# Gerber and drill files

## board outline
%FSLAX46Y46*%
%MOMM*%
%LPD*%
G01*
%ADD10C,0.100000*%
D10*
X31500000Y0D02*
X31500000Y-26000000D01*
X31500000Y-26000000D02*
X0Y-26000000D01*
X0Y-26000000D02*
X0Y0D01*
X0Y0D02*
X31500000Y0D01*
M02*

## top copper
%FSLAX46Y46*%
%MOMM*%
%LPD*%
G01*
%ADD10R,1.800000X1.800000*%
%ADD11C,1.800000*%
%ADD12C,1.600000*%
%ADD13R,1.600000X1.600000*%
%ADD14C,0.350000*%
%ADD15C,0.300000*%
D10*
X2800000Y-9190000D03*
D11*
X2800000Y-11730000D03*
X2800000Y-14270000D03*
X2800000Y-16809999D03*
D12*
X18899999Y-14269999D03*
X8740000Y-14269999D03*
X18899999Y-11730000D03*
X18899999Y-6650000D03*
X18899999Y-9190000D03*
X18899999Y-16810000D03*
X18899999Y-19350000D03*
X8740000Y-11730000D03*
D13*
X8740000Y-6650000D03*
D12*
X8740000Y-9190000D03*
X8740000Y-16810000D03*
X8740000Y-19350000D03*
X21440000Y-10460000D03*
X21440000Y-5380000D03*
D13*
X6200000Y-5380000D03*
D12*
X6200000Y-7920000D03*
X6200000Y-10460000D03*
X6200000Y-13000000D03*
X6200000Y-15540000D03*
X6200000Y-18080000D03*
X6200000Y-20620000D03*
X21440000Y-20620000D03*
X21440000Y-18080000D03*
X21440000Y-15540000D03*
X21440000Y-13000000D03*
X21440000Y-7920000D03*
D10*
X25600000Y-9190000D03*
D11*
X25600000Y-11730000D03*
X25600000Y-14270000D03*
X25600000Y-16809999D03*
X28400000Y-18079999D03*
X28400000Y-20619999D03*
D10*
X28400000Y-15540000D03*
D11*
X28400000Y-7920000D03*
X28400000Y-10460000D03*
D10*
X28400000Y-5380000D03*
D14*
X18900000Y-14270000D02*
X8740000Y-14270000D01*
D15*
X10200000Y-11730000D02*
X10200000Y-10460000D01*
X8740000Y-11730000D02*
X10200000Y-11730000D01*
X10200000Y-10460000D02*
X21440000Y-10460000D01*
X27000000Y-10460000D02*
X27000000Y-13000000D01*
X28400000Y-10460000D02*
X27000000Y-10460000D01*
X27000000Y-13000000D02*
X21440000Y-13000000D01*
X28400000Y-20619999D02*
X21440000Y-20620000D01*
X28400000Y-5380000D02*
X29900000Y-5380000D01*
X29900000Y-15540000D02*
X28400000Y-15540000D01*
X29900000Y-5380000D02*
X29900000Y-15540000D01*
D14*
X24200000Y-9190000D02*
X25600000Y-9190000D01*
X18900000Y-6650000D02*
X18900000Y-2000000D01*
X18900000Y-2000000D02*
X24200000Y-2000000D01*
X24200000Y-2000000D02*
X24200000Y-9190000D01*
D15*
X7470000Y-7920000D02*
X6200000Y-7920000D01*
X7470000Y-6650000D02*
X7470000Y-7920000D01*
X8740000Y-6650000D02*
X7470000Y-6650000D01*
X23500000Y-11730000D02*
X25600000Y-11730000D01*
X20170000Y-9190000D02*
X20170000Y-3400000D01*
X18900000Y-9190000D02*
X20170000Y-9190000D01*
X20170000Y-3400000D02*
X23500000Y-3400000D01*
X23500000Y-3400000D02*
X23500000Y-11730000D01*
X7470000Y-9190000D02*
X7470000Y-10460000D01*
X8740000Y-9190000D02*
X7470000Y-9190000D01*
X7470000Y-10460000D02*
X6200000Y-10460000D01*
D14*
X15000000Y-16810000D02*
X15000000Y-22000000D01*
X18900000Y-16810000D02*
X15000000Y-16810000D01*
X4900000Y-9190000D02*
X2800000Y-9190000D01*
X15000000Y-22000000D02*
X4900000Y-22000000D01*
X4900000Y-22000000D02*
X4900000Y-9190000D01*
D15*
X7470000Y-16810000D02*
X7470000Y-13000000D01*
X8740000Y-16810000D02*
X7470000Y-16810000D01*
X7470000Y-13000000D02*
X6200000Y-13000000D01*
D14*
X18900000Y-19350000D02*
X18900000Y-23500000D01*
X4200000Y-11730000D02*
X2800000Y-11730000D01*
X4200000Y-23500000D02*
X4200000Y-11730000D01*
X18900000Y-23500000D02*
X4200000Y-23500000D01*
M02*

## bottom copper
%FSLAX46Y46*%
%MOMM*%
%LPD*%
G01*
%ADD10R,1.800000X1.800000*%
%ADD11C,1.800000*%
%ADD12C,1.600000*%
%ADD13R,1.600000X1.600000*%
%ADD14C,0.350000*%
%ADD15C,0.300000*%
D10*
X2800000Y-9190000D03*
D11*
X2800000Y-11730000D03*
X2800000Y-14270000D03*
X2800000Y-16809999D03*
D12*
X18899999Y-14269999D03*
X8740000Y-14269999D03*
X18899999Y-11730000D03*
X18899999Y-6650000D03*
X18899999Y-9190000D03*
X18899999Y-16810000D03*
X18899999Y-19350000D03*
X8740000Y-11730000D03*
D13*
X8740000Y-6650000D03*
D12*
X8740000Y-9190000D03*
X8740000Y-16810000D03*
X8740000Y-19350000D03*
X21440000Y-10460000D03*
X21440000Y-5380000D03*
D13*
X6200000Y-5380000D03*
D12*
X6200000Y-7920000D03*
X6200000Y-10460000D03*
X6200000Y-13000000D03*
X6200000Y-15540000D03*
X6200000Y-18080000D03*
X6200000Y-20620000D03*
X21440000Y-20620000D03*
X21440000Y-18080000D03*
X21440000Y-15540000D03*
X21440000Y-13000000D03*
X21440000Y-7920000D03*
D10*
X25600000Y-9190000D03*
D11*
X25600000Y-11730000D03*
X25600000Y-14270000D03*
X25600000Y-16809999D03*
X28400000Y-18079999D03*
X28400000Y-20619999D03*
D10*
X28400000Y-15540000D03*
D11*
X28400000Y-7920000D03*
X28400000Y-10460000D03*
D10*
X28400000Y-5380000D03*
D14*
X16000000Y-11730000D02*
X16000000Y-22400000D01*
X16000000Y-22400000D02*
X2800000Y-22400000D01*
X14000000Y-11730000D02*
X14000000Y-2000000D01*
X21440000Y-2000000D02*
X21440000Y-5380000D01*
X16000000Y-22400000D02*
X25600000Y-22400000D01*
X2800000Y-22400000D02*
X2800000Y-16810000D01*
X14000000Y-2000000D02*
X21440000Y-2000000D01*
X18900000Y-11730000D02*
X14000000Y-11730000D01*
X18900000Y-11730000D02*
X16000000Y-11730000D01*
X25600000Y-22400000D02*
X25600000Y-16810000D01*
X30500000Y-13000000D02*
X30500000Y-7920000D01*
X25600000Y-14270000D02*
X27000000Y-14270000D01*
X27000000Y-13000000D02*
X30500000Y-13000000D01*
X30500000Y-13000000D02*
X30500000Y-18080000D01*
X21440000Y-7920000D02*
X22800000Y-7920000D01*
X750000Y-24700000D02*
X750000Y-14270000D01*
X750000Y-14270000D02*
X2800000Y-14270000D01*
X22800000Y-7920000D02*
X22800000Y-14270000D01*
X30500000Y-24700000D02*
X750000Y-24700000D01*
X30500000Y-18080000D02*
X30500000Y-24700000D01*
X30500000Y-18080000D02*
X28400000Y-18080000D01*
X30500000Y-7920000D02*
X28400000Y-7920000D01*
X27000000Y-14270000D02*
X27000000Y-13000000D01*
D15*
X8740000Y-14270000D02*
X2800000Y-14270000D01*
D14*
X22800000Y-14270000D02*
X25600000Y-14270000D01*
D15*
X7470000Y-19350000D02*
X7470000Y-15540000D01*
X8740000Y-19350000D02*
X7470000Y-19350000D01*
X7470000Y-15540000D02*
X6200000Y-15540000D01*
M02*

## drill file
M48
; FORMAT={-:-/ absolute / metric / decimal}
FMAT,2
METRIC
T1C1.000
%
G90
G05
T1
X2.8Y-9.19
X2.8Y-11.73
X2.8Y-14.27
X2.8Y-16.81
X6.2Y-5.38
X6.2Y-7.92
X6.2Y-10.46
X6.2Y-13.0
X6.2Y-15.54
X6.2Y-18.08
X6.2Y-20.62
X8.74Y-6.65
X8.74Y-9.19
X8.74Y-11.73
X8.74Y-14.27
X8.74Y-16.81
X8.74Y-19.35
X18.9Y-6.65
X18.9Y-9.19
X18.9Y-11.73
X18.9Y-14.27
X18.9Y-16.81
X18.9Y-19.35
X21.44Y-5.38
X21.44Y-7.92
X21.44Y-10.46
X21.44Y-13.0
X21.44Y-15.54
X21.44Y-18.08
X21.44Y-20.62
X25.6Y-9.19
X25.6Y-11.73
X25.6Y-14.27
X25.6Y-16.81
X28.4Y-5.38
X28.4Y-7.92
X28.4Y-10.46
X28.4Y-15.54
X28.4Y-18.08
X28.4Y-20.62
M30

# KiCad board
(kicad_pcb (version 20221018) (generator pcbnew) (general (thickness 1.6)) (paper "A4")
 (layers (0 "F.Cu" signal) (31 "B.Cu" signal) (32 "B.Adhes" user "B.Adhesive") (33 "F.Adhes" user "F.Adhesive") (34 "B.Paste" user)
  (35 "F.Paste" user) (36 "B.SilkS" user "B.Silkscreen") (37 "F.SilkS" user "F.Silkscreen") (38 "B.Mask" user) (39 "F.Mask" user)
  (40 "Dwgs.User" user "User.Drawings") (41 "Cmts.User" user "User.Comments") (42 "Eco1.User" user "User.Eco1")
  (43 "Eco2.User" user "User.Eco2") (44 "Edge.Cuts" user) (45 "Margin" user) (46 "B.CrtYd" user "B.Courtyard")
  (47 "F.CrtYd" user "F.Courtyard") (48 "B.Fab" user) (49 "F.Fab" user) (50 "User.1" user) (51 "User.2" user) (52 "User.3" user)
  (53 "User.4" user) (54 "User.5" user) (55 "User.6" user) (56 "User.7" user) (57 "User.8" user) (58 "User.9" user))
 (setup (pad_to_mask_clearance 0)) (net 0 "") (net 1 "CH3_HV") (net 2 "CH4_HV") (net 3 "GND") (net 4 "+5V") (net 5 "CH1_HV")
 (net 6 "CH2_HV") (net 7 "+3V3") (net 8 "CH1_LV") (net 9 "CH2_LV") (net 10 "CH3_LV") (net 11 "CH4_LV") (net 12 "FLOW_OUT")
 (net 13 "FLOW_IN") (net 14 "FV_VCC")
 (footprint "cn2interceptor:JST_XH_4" (layer "F.Cu") (at 2.8 9.19)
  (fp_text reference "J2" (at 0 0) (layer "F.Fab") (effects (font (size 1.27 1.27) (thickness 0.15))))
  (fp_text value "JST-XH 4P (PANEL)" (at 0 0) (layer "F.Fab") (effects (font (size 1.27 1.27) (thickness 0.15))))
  (pad "1" thru_hole rect (at 0 0) (size 1.8 1.8) (drill 1) (layers "*.Cu" "*.Mask") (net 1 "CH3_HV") (thermal_bridge_angle 45))
  (pad "2" thru_hole circle (at 0 2.54) (size 1.8 1.8) (drill 1) (layers "*.Cu" "*.Mask") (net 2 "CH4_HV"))
  (pad "3" thru_hole circle (at 0 5.08) (size 1.8 1.8) (drill 1) (layers "*.Cu" "*.Mask") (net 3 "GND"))
  (pad "4" thru_hole circle (at 0 7.619999) (size 1.8 1.8) (drill 1) (layers "*.Cu" "*.Mask") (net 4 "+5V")))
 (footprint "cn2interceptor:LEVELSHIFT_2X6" (layer "F.Cu") (at 8.74 6.65)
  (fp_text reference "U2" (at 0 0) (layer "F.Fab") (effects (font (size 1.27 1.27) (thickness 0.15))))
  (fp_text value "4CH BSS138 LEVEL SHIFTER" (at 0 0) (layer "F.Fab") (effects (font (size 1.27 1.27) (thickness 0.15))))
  (pad "GND_H" thru_hole circle (at 10.159999 7.619999) (size 1.6 1.6) (drill 1) (layers "*.Cu" "*.Mask") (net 3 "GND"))
  (pad "GND_L" thru_hole circle (at 0 7.619999) (size 1.6 1.6) (drill 1) (layers "*.Cu" "*.Mask") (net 3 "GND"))
  (pad "HV" thru_hole circle (at 10.159999 5.08) (size 1.6 1.6) (drill 1) (layers "*.Cu" "*.Mask") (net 4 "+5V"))
  (pad "HV1" thru_hole circle (at 10.159999 0) (size 1.6 1.6) (drill 1) (layers "*.Cu" "*.Mask") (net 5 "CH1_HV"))
  (pad "HV2" thru_hole circle (at 10.159999 2.54) (size 1.6 1.6) (drill 1) (layers "*.Cu" "*.Mask") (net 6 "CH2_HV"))
  (pad "HV3" thru_hole circle (at 10.159999 10.16) (size 1.6 1.6) (drill 1) (layers "*.Cu" "*.Mask") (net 1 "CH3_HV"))
  (pad "HV4" thru_hole circle (at 10.159999 12.7) (size 1.6 1.6) (drill 1) (layers "*.Cu" "*.Mask") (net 2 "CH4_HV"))
  (pad "LV" thru_hole circle (at 0 5.08) (size 1.6 1.6) (drill 1) (layers "*.Cu" "*.Mask") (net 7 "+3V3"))
  (pad "LV1" thru_hole rect (at 0 0) (size 1.6 1.6) (drill 1) (layers "*.Cu" "*.Mask") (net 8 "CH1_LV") (thermal_bridge_angle 45))
  (pad "LV2" thru_hole circle (at 0 2.54) (size 1.6 1.6) (drill 1) (layers "*.Cu" "*.Mask") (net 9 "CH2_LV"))
  (pad "LV3" thru_hole circle (at 0 10.16) (size 1.6 1.6) (drill 1) (layers "*.Cu" "*.Mask") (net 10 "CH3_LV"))
  (pad "LV4" thru_hole circle (at 0 12.7) (size 1.6 1.6) (drill 1) (layers "*.Cu" "*.Mask") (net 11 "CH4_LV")))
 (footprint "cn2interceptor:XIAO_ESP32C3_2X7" (layer "F.Cu") (at 6.2 5.38)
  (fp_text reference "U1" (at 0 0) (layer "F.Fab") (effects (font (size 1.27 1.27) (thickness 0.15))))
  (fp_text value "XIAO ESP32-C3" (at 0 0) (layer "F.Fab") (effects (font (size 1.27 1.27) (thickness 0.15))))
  (pad "3V3" thru_hole circle (at 15.24 5.08) (size 1.6 1.6) (drill 1) (layers "*.Cu" "*.Mask") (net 7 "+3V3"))
  (pad "5V" thru_hole circle (at 15.24 0) (size 1.6 1.6) (drill 1) (layers "*.Cu" "*.Mask") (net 4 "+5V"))
  (pad "D0" thru_hole rect (at 0 0) (size 1.6 1.6) (drill 1) (layers "*.Cu" "*.Mask") (thermal_bridge_angle 45))
  (pad "D1" thru_hole circle (at 0 2.54) (size 1.6 1.6) (drill 1) (layers "*.Cu" "*.Mask") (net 8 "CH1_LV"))
  (pad "D2" thru_hole circle (at 0 5.08) (size 1.6 1.6) (drill 1) (layers "*.Cu" "*.Mask") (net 9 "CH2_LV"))
  (pad "D3" thru_hole circle (at 0 7.62) (size 1.6 1.6) (drill 1) (layers "*.Cu" "*.Mask") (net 10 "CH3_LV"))
  (pad "D4" thru_hole circle (at 0 10.16) (size 1.6 1.6) (drill 1) (layers "*.Cu" "*.Mask") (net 11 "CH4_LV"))
  (pad "D5" thru_hole circle (at 0 12.7) (size 1.6 1.6) (drill 1) (layers "*.Cu" "*.Mask"))
  (pad "D6" thru_hole circle (at 0 15.24) (size 1.6 1.6) (drill 1) (layers "*.Cu" "*.Mask"))
  (pad "D7" thru_hole circle (at 15.24 15.24) (size 1.6 1.6) (drill 1) (layers "*.Cu" "*.Mask") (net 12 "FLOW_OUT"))
  (pad "D8" thru_hole circle (at 15.24 12.7) (size 1.6 1.6) (drill 1) (layers "*.Cu" "*.Mask"))
  (pad "D9" thru_hole circle (at 15.24 10.16) (size 1.6 1.6) (drill 1) (layers "*.Cu" "*.Mask"))
  (pad "D10" thru_hole circle (at 15.24 7.62) (size 1.6 1.6) (drill 1) (layers "*.Cu" "*.Mask") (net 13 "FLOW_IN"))
  (pad "GND" thru_hole circle (at 15.24 2.54) (size 1.6 1.6) (drill 1) (layers "*.Cu" "*.Mask") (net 3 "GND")))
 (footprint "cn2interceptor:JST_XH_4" (layer "F.Cu") (at 25.6 9.19)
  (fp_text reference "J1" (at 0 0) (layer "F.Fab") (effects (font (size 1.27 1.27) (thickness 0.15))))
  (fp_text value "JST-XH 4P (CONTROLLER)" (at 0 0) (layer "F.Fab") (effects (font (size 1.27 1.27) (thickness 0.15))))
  (pad "1" thru_hole rect (at 0 0) (size 1.8 1.8) (drill 1) (layers "*.Cu" "*.Mask") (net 5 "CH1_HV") (thermal_bridge_angle 45))
  (pad "2" thru_hole circle (at 0 2.54) (size 1.8 1.8) (drill 1) (layers "*.Cu" "*.Mask") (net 6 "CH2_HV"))
  (pad "3" thru_hole circle (at 0 5.08) (size 1.8 1.8) (drill 1) (layers "*.Cu" "*.Mask") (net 3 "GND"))
  (pad "4" thru_hole circle (at 0 7.619999) (size 1.8 1.8) (drill 1) (layers "*.Cu" "*.Mask") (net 4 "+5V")))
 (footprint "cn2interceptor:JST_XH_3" (layer "F.Cu") (at 28.4 15.54)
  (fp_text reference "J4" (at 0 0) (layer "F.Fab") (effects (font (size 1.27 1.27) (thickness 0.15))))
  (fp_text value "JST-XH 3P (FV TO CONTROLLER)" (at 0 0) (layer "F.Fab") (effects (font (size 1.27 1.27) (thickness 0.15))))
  (pad "GND" thru_hole circle (at 0 2.539999) (size 1.8 1.8) (drill 1) (layers "*.Cu" "*.Mask") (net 3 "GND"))
  (pad "SIG" thru_hole circle (at 0 5.079999) (size 1.8 1.8) (drill 1) (layers "*.Cu" "*.Mask") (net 12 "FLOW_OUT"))
  (pad "VCC" thru_hole rect (at 0 0) (size 1.8 1.8) (drill 1) (layers "*.Cu" "*.Mask") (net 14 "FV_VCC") (thermal_bridge_angle 45)))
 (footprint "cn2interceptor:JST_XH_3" (layer "F.Cu") (at 28.4 5.38)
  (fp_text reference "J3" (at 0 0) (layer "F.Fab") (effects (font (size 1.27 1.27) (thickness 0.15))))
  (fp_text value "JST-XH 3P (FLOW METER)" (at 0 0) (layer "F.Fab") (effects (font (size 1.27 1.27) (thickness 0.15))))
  (pad "GND" thru_hole circle (at 0 2.54) (size 1.8 1.8) (drill 1) (layers "*.Cu" "*.Mask") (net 3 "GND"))
  (pad "SIG" thru_hole circle (at 0 5.08) (size 1.8 1.8) (drill 1) (layers "*.Cu" "*.Mask") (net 13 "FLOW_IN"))
  (pad "VCC" thru_hole rect (at 0 0) (size 1.8 1.8) (drill 1) (layers "*.Cu" "*.Mask") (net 14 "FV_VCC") (thermal_bridge_angle 45)))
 (gr_line (start 31.5 0) (end 31.5 26) (stroke (width 0.1) (type default)) (layer "Edge.Cuts"))
 (gr_line (start 31.5 26) (end 0 26) (stroke (width 0.1) (type default)) (layer "Edge.Cuts"))
 (gr_line (start 0 26) (end 0 0) (stroke (width 0.1) (type default)) (layer "Edge.Cuts"))
 (gr_line (start 0 0) (end 31.5 0) (stroke (width 0.1) (type default)) (layer "Edge.Cuts"))
 (segment (start 16 11.73) (end 16 22.4) (width 0.35) (layer "B.Cu") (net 4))
 (segment (start 16 22.4) (end 2.8 22.4) (width 0.35) (layer "B.Cu") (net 4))
 (segment (start 14 11.73) (end 14 2) (width 0.35) (layer "B.Cu") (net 4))
 (segment (start 21.44 2) (end 21.44 5.38) (width 0.35) (layer "B.Cu") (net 4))
 (segment (start 16 22.4) (end 25.6 22.4) (width 0.35) (layer "B.Cu") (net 4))
 (segment (start 2.8 22.4) (end 2.8 16.81) (width 0.35) (layer "B.Cu") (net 4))
 (segment (start 14 2) (end 21.44 2) (width 0.35) (layer "B.Cu") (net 4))
 (segment (start 18.9 11.73) (end 14 11.73) (width 0.35) (layer "B.Cu") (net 4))
 (segment (start 18.9 11.73) (end 16 11.73) (width 0.35) (layer "B.Cu") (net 4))
 (segment (start 25.6 22.4) (end 25.6 16.81) (width 0.35) (layer "B.Cu") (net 4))
 (segment (start 18.9 14.27) (end 8.74 14.27) (width 0.35) (layer "F.Cu") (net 3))
 (segment (start 30.5 13) (end 30.5 7.92) (width 0.35) (layer "B.Cu") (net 3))
 (segment (start 25.6 14.27) (end 27 14.27) (width 0.35) (layer "B.Cu") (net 3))
 (segment (start 27 13) (end 30.5 13) (width 0.35) (layer "B.Cu") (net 3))
 (segment (start 30.5 13) (end 30.5 18.08) (width 0.35) (layer "B.Cu") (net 3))
 (segment (start 21.44 7.92) (end 22.8 7.92) (width 0.35) (layer "B.Cu") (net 3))
 (segment (start 0.75 24.7) (end 0.75 14.27) (width 0.35) (layer "B.Cu") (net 3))
 (segment (start 0.75 14.27) (end 2.8 14.27) (width 0.35) (layer "B.Cu") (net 3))
 (segment (start 22.8 7.92) (end 22.8 14.27) (width 0.35) (layer "B.Cu") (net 3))
 (segment (start 30.5 24.7) (end 0.75 24.7) (width 0.35) (layer "B.Cu") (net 3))
 (segment (start 30.5 18.08) (end 30.5 24.7) (width 0.35) (layer "B.Cu") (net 3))
 (segment (start 30.5 18.08) (end 28.4 18.08) (width 0.35) (layer "B.Cu") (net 3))
 (segment (start 30.5 7.92) (end 28.4 7.92) (width 0.35) (layer "B.Cu") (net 3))
 (segment (start 27 14.27) (end 27 13) (width 0.35) (layer "B.Cu") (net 3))
 (segment (start 8.74 14.27) (end 2.8 14.27) (width 0.3) (layer "B.Cu") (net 3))
 (segment (start 22.8 14.27) (end 25.6 14.27) (width 0.35) (layer "B.Cu") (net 3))
 (segment (start 10.2 11.73) (end 10.2 10.46) (width 0.3) (layer "F.Cu") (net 7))
 (segment (start 8.74 11.73) (end 10.2 11.73) (width 0.3) (layer "F.Cu") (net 7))
 (segment (start 10.2 10.46) (end 21.44 10.46) (width 0.3) (layer "F.Cu") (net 7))
 (segment (start 27 10.46) (end 27 13) (width 0.3) (layer "F.Cu") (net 13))
 (segment (start 28.4 10.46) (end 27 10.46) (width 0.3) (layer "F.Cu") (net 13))
 (segment (start 27 13) (end 21.44 13) (width 0.3) (layer "F.Cu") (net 13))
 (segment (start 28.4 20.619999) (end 21.44 20.62) (width 0.3) (layer "F.Cu") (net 12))
 (segment (start 28.4 5.38) (end 29.9 5.38) (width 0.3) (layer "F.Cu") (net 14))
 (segment (start 29.9 15.54) (end 28.4 15.54) (width 0.3) (layer "F.Cu") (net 14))
 (segment (start 29.9 5.38) (end 29.9 15.54) (width 0.3) (layer "F.Cu") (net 14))
 (segment (start 24.2 9.19) (end 25.6 9.19) (width 0.35) (layer "F.Cu") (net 5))
 (segment (start 18.9 6.65) (end 18.9 2) (width 0.35) (layer "F.Cu") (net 5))
 (segment (start 18.9 2) (end 24.2 2) (width 0.35) (layer "F.Cu") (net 5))
 (segment (start 24.2 2) (end 24.2 9.19) (width 0.35) (layer "F.Cu") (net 5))
 (segment (start 7.47 7.92) (end 6.2 7.92) (width 0.3) (layer "F.Cu") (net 8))
 (segment (start 7.47 6.65) (end 7.47 7.92) (width 0.3) (layer "F.Cu") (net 8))
 (segment (start 8.74 6.65) (end 7.47 6.65) (width 0.3) (layer "F.Cu") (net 8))
 (segment (start 23.5 11.73) (end 25.6 11.73) (width 0.3) (layer "F.Cu") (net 6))
 (segment (start 20.17 9.19) (end 20.17 3.4) (width 0.3) (layer "F.Cu") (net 6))
 (segment (start 18.9 9.19) (end 20.17 9.19) (width 0.3) (layer "F.Cu") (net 6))
 (segment (start 20.17 3.4) (end 23.5 3.4) (width 0.3) (layer "F.Cu") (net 6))
 (segment (start 23.5 3.4) (end 23.5 11.73) (width 0.3) (layer "F.Cu") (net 6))
 (segment (start 7.47 9.19) (end 7.47 10.46) (width 0.3) (layer "F.Cu") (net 9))
 (segment (start 8.74 9.19) (end 7.47 9.19) (width 0.3) (layer "F.Cu") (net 9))
 (segment (start 7.47 10.46) (end 6.2 10.46) (width 0.3) (layer "F.Cu") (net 9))
 (segment (start 15 16.81) (end 15 22) (width 0.35) (layer "F.Cu") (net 1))
 (segment (start 18.9 16.81) (end 15 16.81) (width 0.35) (layer "F.Cu") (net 1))
 (segment (start 4.9 9.19) (end 2.8 9.19) (width 0.35) (layer "F.Cu") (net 1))
 (segment (start 15 22) (end 4.9 22) (width 0.35) (layer "F.Cu") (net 1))
 (segment (start 4.9 22) (end 4.9 9.19) (width 0.35) (layer "F.Cu") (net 1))
 (segment (start 7.47 16.81) (end 7.47 13) (width 0.3) (layer "F.Cu") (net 10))
 (segment (start 8.74 16.81) (end 7.47 16.81) (width 0.3) (layer "F.Cu") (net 10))
 (segment (start 7.47 13) (end 6.2 13) (width 0.3) (layer "F.Cu") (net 10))
 (segment (start 18.9 19.35) (end 18.9 23.5) (width 0.35) (layer "F.Cu") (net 2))
 (segment (start 4.2 11.73) (end 2.8 11.73) (width 0.35) (layer "F.Cu") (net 2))
 (segment (start 4.2 23.5) (end 4.2 11.73) (width 0.35) (layer "F.Cu") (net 2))
 (segment (start 18.9 23.5) (end 4.2 23.5) (width 0.35) (layer "F.Cu") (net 2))
 (segment (start 7.47 19.35) (end 7.47 15.54) (width 0.3) (layer "B.Cu") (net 11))
 (segment (start 8.74 19.35) (end 7.47 19.35) (width 0.3) (layer "B.Cu") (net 11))
 (segment (start 7.47 15.54) (end 6.2 15.54) (width 0.3) (layer "B.Cu") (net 11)))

